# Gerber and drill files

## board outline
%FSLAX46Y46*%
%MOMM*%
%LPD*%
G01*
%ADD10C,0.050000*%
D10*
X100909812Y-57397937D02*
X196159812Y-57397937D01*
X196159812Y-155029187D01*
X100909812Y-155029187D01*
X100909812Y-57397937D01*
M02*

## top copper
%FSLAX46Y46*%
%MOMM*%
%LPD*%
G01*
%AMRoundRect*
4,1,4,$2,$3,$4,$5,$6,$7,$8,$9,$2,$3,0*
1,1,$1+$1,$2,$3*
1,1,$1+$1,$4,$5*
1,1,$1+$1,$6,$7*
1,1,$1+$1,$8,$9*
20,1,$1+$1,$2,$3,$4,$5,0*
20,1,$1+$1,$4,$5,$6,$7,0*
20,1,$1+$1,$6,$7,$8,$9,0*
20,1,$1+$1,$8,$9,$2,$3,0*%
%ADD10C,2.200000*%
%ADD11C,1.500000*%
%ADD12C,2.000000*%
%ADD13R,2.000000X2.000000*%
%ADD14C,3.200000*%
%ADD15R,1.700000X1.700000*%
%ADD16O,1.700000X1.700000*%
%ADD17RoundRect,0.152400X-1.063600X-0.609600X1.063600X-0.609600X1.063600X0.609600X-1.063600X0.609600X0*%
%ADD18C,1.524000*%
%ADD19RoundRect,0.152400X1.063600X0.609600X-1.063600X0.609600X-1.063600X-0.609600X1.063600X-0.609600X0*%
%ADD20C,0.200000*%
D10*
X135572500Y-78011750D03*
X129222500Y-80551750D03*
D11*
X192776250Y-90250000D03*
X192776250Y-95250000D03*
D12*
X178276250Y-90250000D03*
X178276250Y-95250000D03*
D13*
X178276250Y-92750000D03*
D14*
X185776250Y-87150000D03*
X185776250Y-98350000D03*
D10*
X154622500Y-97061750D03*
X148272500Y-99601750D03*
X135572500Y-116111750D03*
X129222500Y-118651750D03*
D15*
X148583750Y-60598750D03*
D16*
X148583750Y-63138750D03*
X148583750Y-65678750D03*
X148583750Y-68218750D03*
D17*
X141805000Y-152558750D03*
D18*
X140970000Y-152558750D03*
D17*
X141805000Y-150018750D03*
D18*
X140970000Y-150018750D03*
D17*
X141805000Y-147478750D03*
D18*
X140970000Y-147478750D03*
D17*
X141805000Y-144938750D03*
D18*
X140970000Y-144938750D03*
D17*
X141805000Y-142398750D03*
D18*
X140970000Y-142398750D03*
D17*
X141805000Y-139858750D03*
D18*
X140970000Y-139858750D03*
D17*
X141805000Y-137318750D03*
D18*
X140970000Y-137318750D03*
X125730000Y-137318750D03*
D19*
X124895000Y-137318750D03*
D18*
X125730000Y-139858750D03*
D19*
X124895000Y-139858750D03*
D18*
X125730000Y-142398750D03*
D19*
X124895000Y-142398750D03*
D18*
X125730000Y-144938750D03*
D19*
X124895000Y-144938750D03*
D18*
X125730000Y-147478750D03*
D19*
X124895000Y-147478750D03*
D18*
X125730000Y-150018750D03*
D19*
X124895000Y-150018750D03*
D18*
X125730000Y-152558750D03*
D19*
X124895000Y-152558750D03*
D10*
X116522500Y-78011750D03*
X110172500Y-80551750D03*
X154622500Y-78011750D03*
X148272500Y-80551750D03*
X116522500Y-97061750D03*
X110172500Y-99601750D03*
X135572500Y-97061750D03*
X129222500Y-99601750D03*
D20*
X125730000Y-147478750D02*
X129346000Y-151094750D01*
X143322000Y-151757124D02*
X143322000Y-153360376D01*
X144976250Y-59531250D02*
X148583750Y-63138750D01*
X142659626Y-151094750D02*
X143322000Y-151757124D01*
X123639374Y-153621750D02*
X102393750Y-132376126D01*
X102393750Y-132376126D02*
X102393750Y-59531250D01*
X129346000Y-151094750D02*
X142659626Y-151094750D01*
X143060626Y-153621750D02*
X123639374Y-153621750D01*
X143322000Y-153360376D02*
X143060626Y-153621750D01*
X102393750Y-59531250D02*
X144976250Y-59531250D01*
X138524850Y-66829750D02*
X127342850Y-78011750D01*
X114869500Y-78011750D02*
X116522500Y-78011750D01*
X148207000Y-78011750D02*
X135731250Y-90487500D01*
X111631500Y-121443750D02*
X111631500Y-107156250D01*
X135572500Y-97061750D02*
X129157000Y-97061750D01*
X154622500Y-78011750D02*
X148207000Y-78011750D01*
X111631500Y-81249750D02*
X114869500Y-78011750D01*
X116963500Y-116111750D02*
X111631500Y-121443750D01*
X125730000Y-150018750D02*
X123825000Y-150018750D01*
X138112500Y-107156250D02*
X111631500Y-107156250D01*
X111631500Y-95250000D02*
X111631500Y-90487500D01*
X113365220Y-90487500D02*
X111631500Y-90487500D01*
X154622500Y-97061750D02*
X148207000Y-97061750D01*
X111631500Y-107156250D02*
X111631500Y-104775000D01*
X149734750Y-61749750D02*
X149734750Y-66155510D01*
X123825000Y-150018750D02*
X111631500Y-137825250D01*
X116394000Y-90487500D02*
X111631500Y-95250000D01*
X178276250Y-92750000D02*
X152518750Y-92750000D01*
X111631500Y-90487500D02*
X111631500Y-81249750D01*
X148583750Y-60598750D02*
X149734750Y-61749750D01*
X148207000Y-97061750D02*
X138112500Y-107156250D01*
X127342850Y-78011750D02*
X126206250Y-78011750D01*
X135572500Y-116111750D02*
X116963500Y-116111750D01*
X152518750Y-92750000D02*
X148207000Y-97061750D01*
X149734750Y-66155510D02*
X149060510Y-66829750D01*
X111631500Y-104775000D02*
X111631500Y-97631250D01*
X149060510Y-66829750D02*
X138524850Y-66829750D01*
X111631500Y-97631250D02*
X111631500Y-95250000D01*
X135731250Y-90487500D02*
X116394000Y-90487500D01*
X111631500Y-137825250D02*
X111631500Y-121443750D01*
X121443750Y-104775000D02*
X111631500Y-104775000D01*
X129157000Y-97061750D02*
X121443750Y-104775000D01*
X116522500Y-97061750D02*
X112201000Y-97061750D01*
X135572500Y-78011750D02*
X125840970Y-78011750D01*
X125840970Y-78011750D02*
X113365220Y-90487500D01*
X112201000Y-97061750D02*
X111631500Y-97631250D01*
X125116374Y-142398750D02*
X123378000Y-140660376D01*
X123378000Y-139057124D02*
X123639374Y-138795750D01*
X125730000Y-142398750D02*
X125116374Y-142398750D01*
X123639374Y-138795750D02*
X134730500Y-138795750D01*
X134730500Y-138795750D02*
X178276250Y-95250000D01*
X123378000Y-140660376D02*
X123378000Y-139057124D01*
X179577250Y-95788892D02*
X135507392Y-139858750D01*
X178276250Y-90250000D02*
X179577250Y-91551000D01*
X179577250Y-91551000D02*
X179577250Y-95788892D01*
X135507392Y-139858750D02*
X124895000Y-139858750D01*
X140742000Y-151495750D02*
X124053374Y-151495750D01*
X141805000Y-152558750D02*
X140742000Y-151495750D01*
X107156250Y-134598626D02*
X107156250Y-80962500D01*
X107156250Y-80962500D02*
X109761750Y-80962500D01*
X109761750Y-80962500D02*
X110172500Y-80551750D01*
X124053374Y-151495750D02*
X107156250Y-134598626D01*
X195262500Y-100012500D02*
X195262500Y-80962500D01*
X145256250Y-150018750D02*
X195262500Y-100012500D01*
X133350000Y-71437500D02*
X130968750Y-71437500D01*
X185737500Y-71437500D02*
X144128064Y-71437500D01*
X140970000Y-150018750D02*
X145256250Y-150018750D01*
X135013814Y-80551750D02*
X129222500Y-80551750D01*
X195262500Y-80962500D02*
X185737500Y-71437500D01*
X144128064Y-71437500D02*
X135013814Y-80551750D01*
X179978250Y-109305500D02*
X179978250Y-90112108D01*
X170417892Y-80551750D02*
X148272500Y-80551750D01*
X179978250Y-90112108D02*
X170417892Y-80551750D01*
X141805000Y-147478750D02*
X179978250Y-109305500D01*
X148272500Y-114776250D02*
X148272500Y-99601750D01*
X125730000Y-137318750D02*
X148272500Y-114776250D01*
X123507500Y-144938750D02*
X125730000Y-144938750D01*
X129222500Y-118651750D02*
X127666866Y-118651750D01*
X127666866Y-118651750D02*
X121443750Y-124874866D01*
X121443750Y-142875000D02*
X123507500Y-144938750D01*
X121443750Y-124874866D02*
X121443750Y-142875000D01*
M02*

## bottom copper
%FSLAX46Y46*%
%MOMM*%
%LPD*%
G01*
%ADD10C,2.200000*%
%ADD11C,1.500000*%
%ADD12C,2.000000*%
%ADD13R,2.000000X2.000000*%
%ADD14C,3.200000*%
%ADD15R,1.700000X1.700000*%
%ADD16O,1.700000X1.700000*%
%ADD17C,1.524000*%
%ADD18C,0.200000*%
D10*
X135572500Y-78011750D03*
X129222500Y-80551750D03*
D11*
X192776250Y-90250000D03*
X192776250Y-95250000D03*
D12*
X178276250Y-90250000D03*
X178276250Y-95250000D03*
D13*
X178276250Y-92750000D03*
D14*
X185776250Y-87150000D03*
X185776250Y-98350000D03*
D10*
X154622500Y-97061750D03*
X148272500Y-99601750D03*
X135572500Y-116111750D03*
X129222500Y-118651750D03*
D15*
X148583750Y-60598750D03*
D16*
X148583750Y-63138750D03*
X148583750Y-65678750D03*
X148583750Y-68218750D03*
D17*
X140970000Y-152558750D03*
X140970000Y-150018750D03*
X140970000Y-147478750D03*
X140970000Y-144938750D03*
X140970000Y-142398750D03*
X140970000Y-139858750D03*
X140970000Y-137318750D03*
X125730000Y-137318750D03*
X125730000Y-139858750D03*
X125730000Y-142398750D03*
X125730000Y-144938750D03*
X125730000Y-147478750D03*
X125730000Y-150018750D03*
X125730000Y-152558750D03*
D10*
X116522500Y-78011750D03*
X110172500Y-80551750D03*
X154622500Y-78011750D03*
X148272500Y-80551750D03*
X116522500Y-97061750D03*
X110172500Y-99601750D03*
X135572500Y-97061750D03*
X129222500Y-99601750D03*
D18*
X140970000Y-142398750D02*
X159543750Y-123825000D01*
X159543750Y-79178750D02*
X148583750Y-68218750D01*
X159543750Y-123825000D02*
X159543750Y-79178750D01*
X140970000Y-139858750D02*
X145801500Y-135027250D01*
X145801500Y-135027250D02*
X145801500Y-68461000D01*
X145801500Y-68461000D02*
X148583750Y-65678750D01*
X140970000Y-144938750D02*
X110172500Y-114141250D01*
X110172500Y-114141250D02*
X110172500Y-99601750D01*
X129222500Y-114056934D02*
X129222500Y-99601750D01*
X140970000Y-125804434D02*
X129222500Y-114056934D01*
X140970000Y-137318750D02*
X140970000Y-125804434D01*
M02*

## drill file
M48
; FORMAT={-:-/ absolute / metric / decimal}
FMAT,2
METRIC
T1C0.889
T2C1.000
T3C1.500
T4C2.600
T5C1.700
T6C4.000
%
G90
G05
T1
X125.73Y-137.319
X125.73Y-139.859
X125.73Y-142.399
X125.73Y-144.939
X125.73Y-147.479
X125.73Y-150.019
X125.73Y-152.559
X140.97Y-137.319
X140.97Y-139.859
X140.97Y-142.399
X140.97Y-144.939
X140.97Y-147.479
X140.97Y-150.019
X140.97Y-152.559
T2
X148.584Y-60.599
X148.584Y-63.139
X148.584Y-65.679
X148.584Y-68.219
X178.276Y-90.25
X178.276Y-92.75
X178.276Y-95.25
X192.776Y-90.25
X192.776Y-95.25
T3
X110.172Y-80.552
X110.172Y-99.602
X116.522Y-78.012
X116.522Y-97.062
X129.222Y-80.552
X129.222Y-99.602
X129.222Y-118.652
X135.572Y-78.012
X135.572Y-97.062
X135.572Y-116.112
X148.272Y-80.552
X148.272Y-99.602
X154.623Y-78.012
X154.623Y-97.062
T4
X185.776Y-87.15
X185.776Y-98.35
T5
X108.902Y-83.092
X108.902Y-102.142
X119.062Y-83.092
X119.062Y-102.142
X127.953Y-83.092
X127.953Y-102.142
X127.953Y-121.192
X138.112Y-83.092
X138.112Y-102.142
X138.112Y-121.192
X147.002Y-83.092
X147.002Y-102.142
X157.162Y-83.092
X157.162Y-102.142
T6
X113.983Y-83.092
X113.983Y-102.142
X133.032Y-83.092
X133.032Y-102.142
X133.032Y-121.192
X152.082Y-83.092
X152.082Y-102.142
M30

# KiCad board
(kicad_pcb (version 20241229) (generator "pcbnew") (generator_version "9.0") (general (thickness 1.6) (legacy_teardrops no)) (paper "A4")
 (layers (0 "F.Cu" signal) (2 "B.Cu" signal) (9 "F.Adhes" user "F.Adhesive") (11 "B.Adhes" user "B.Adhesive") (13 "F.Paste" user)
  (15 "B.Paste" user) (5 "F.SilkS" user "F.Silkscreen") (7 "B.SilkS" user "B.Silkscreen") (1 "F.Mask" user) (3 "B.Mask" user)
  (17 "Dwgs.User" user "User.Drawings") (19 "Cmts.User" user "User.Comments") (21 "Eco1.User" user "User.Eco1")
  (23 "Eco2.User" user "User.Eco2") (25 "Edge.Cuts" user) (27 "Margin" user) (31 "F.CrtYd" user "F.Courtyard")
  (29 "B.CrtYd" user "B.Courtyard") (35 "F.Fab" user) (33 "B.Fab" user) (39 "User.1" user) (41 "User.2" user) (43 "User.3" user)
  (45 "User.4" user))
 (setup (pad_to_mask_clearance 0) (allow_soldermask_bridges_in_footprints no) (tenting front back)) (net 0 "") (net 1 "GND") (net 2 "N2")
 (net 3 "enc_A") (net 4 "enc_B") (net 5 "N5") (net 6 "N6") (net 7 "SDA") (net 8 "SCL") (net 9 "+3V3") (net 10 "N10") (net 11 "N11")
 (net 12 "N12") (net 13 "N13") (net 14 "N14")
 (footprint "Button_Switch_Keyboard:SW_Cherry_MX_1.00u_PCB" (layer "F.Cu") (at 135.5725 78.01175)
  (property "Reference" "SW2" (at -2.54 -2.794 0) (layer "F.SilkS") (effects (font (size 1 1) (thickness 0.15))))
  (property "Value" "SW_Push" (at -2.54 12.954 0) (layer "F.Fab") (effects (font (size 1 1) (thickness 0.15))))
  (pad "" np_thru_hole circle (at -7.62 5.08) (size 1.7 1.7) (drill 1.7) (layers "*.Cu" "*.Mask"))
  (pad "" np_thru_hole circle (at -2.54 5.08) (size 4 4) (drill 4) (layers "*.Cu" "*.Mask"))
  (pad "" np_thru_hole circle (at 2.54 5.08) (size 1.7 1.7) (drill 1.7) (layers "*.Cu" "*.Mask"))
  (pad "1" thru_hole circle (at 0 0) (size 2.2 2.2) (drill 1.5) (layers "*.Cu" "*.Mask") (remove_unused_layers no) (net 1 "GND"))
  (pad "2" thru_hole circle (at -6.35 2.54) (size 2.2 2.2) (drill 1.5) (layers "*.Cu" "*.Mask") (remove_unused_layers no) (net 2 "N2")))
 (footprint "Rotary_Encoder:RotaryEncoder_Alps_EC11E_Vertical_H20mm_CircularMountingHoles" (layer "F.Cu") (at 178.27625 90.25)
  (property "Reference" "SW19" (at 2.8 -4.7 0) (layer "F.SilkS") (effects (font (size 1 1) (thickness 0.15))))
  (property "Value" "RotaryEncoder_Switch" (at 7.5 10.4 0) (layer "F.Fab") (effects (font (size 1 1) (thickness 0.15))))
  (pad "" thru_hole circle (at 14.5 0) (size 1.5 1.5) (drill 1) (layers "*.Cu" "*.Mask") (remove_unused_layers no))
  (pad "" thru_hole circle (at 14.5 5) (size 1.5 1.5) (drill 1) (layers "*.Cu" "*.Mask") (remove_unused_layers no))
  (pad "A" thru_hole circle (at 0 0) (size 2 2) (drill 1) (layers "*.Cu" "*.Mask") (remove_unused_layers no) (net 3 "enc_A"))
  (pad "B" thru_hole circle (at 0 5) (size 2 2) (drill 1) (layers "*.Cu" "*.Mask") (remove_unused_layers no) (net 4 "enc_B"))
  (pad "C" thru_hole rect (at 0 2.5) (size 2 2) (drill 1) (layers "*.Cu" "*.Mask") (remove_unused_layers no) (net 1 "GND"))
  (pad "MP" thru_hole circle (at 7.5 -3.1) (size 3.2 3.2) (drill 2.6) (layers "*.Cu" "*.Mask") (remove_unused_layers no))
  (pad "MP" thru_hole circle (at 7.5 8.1) (size 3.2 3.2) (drill 2.6) (layers "*.Cu" "*.Mask") (remove_unused_layers no)))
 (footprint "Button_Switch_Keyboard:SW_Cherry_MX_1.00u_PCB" (layer "F.Cu") (at 154.6225 97.06175)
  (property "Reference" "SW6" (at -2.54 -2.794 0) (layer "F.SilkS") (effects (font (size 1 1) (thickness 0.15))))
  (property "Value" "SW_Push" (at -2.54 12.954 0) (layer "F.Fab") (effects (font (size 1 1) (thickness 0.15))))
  (pad "" np_thru_hole circle (at -7.62 5.08) (size 1.7 1.7) (drill 1.7) (layers "*.Cu" "*.Mask"))
  (pad "" np_thru_hole circle (at -2.54 5.08) (size 4 4) (drill 4) (layers "*.Cu" "*.Mask"))
  (pad "" np_thru_hole circle (at 2.54 5.08) (size 1.7 1.7) (drill 1.7) (layers "*.Cu" "*.Mask"))
  (pad "1" thru_hole circle (at 0 0) (size 2.2 2.2) (drill 1.5) (layers "*.Cu" "*.Mask") (remove_unused_layers no) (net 1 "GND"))
  (pad "2" thru_hole circle (at -6.35 2.54) (size 2.2 2.2) (drill 1.5) (layers "*.Cu" "*.Mask") (remove_unused_layers no) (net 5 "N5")))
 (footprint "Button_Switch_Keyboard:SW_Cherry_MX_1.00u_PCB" (layer "F.Cu") (at 135.5725 116.11175)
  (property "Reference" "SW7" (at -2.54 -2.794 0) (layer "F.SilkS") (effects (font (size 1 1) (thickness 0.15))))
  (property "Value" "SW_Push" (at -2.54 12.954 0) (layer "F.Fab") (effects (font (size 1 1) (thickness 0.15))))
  (pad "" np_thru_hole circle (at -7.62 5.08) (size 1.7 1.7) (drill 1.7) (layers "*.Cu" "*.Mask"))
  (pad "" np_thru_hole circle (at -2.54 5.08) (size 4 4) (drill 4) (layers "*.Cu" "*.Mask"))
  (pad "" np_thru_hole circle (at 2.54 5.08) (size 1.7 1.7) (drill 1.7) (layers "*.Cu" "*.Mask"))
  (pad "1" thru_hole circle (at 0 0) (size 2.2 2.2) (drill 1.5) (layers "*.Cu" "*.Mask") (remove_unused_layers no) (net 1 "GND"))
  (pad "2" thru_hole circle (at -6.35 2.54) (size 2.2 2.2) (drill 1.5) (layers "*.Cu" "*.Mask") (remove_unused_layers no) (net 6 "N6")))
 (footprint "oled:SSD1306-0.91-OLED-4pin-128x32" (layer "F.Cu") (at 112.08375 58.40875)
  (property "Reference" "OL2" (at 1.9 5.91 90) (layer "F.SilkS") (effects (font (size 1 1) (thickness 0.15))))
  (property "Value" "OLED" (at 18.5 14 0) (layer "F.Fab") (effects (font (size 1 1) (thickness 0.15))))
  (pad "1" thru_hole rect (at 36.5 2.19) (size 1.7 1.7) (drill 1) (layers "*.Cu" "*.Mask") (remove_unused_layers no) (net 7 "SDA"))
  (pad "2" thru_hole oval (at 36.5 4.73) (size 1.7 1.7) (drill 1) (layers "*.Cu" "*.Mask") (remove_unused_layers no) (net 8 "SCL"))
  (pad "3" thru_hole oval (at 36.5 7.27) (size 1.7 1.7) (drill 1) (layers "*.Cu" "*.Mask") (remove_unused_layers no) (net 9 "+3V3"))
  (pad "4" thru_hole oval (at 36.5 9.81) (size 1.7 1.7) (drill 1) (layers "*.Cu" "*.Mask") (remove_unused_layers no) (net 1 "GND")))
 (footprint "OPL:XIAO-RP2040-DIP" (layer "F.Cu") (at 133.35 144.93875 180)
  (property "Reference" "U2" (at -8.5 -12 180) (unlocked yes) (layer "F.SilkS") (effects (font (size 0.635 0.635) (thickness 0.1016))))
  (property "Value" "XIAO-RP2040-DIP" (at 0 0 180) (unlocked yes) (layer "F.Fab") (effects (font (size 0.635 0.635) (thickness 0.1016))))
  (pad "1" smd roundrect (at -8.455 -7.62) (size 2.432 1.524) (layers "F.Cu" "F.Mask") (roundrect_rratio 0.1) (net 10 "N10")
   (thermal_bridge_angle 45))
  (pad "1" thru_hole circle (at -7.62 -7.62) (size 1.524 1.524) (drill 0.889) (layers "*.Cu" "*.Mask") (remove_unused_layers no)
   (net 10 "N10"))
  (pad "2" smd roundrect (at -8.455 -5.08) (size 2.432 1.524) (layers "F.Cu" "F.Mask") (roundrect_rratio 0.1) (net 2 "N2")
   (thermal_bridge_angle 45))
  (pad "2" thru_hole circle (at -7.62 -5.08) (size 1.524 1.524) (drill 0.889) (layers "*.Cu" "*.Mask") (remove_unused_layers no)
   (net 2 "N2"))
  (pad "3" smd roundrect (at -8.455 -2.54) (size 2.432 1.524) (layers "F.Cu" "F.Mask") (roundrect_rratio 0.1) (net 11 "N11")
   (thermal_bridge_angle 45))
  (pad "3" thru_hole circle (at -7.62 -2.54) (size 1.524 1.524) (drill 0.889) (layers "*.Cu" "*.Mask") (remove_unused_layers no)
   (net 11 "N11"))
  (pad "4" smd roundrect (at -8.455 0) (size 2.432 1.524) (layers "F.Cu" "F.Mask") (roundrect_rratio 0.1) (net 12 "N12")
   (thermal_bridge_angle 45))
  (pad "4" thru_hole circle (at -7.62 0) (size 1.524 1.524) (drill 0.889) (layers "*.Cu" "*.Mask") (remove_unused_layers no) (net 12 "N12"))
  (pad "5" smd roundrect (at -8.455 2.54) (size 2.432 1.524) (layers "F.Cu" "F.Mask") (roundrect_rratio 0.1) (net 7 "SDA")
   (thermal_bridge_angle 45))
  (pad "5" thru_hole circle (at -7.62 2.54) (size 1.524 1.524) (drill 0.889) (layers "*.Cu" "*.Mask") (remove_unused_layers no)
   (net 7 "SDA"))
  (pad "6" smd roundrect (at -8.455 5.08) (size 2.432 1.524) (layers "F.Cu" "F.Mask") (roundrect_rratio 0.1) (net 8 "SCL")
   (thermal_bridge_angle 45))
  (pad "6" thru_hole circle (at -7.62 5.08) (size 1.524 1.524) (drill 0.889) (layers "*.Cu" "*.Mask") (remove_unused_layers no)
   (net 8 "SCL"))
  (pad "7" smd roundrect (at -8.455 7.62) (size 2.432 1.524) (layers "F.Cu" "F.Mask") (roundrect_rratio 0.1) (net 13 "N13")
   (thermal_bridge_angle 45))
  (pad "7" thru_hole circle (at -7.62 7.62) (size 1.524 1.524) (drill 0.889) (layers "*.Cu" "*.Mask") (remove_unused_layers no)
   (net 13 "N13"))
  (pad "8" thru_hole circle (at 7.62 7.62 180) (size 1.524 1.524) (drill 0.889) (layers "*.Cu" "*.Mask") (remove_unused_layers no)
   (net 5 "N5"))
  (pad "8" smd roundrect (at 8.455 7.62 180) (size 2.432 1.524) (layers "F.Cu" "F.Mask") (roundrect_rratio 0.1) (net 5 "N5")
   (thermal_bridge_angle 45))
  (pad "9" thru_hole circle (at 7.62 5.08 180) (size 1.524 1.524) (drill 0.889) (layers "*.Cu" "*.Mask") (remove_unused_layers no)
   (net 3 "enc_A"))
  (pad "9" smd roundrect (at 8.455 5.08 180) (size 2.432 1.524) (layers "F.Cu" "F.Mask") (roundrect_rratio 0.1) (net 3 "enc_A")
   (thermal_bridge_angle 45))
  (pad "10" thru_hole circle (at 7.62 2.54 180) (size 1.524 1.524) (drill 0.889) (layers "*.Cu" "*.Mask") (remove_unused_layers no)
   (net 4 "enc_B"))
  (pad "10" smd roundrect (at 8.455 2.54 180) (size 2.432 1.524) (layers "F.Cu" "F.Mask") (roundrect_rratio 0.1) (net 4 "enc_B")
   (thermal_bridge_angle 45))
  (pad "11" thru_hole circle (at 7.62 0 180) (size 1.524 1.524) (drill 0.889) (layers "*.Cu" "*.Mask") (remove_unused_layers no)
   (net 6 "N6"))
  (pad "11" smd roundrect (at 8.455 0 180) (size 2.432 1.524) (layers "F.Cu" "F.Mask") (roundrect_rratio 0.1) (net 6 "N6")
   (thermal_bridge_angle 45))
  (pad "12" thru_hole circle (at 7.62 -2.54 180) (size 1.524 1.524) (drill 0.889) (layers "*.Cu" "*.Mask") (remove_unused_layers no)
   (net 9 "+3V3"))
  (pad "12" smd roundrect (at 8.455 -2.54 180) (size 2.432 1.524) (layers "F.Cu" "F.Mask") (roundrect_rratio 0.1) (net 9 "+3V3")
   (thermal_bridge_angle 45))
  (pad "13" thru_hole circle (at 7.62 -5.08 180) (size 1.524 1.524) (drill 0.889) (layers "*.Cu" "*.Mask") (remove_unused_layers no)
   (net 1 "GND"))
  (pad "13" smd roundrect (at 8.455 -5.08 180) (size 2.432 1.524) (layers "F.Cu" "F.Mask") (roundrect_rratio 0.1) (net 1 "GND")
   (thermal_bridge_angle 45))
  (pad "14" thru_hole circle (at 7.62 -7.62 180) (size 1.524 1.524) (drill 0.889) (layers "*.Cu" "*.Mask") (remove_unused_layers no)
   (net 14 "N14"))
  (pad "14" smd roundrect (at 8.455 -7.62 180) (size 2.432 1.524) (layers "F.Cu" "F.Mask") (roundrect_rratio 0.1) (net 14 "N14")
   (thermal_bridge_angle 45)))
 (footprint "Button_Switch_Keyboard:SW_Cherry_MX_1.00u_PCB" (layer "F.Cu") (at 116.5225 78.01175)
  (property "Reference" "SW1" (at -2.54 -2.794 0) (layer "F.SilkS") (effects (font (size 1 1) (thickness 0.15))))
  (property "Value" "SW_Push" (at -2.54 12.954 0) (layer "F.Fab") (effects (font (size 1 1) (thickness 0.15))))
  (pad "" np_thru_hole circle (at -7.62 5.08) (size 1.7 1.7) (drill 1.7) (layers "*.Cu" "*.Mask"))
  (pad "" np_thru_hole circle (at -2.54 5.08) (size 4 4) (drill 4) (layers "*.Cu" "*.Mask"))
  (pad "" np_thru_hole circle (at 2.54 5.08) (size 1.7 1.7) (drill 1.7) (layers "*.Cu" "*.Mask"))
  (pad "1" thru_hole circle (at 0 0) (size 2.2 2.2) (drill 1.5) (layers "*.Cu" "*.Mask") (remove_unused_layers no) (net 1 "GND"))
  (pad "2" thru_hole circle (at -6.35 2.54) (size 2.2 2.2) (drill 1.5) (layers "*.Cu" "*.Mask") (remove_unused_layers no) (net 10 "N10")))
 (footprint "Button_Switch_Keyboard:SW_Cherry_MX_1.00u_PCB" (layer "F.Cu") (at 154.6225 78.01175)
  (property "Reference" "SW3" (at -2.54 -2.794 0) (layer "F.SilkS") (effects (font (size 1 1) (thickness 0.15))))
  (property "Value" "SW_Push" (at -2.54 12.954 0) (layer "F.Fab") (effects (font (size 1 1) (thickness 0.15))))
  (pad "" np_thru_hole circle (at -7.62 5.08) (size 1.7 1.7) (drill 1.7) (layers "*.Cu" "*.Mask"))
  (pad "" np_thru_hole circle (at -2.54 5.08) (size 4 4) (drill 4) (layers "*.Cu" "*.Mask"))
  (pad "" np_thru_hole circle (at 2.54 5.08) (size 1.7 1.7) (drill 1.7) (layers "*.Cu" "*.Mask"))
  (pad "1" thru_hole circle (at 0 0) (size 2.2 2.2) (drill 1.5) (layers "*.Cu" "*.Mask") (remove_unused_layers no) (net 1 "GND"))
  (pad "2" thru_hole circle (at -6.35 2.54) (size 2.2 2.2) (drill 1.5) (layers "*.Cu" "*.Mask") (remove_unused_layers no) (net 11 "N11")))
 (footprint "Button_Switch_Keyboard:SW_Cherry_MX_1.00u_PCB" (layer "F.Cu") (at 116.5225 97.06175)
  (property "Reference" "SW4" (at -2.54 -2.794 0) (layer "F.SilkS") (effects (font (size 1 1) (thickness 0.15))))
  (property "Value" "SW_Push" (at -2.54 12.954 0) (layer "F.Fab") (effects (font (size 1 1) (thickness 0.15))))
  (pad "" np_thru_hole circle (at -7.62 5.08) (size 1.7 1.7) (drill 1.7) (layers "*.Cu" "*.Mask"))
  (pad "" np_thru_hole circle (at -2.54 5.08) (size 4 4) (drill 4) (layers "*.Cu" "*.Mask"))
  (pad "" np_thru_hole circle (at 2.54 5.08) (size 1.7 1.7) (drill 1.7) (layers "*.Cu" "*.Mask"))
  (pad "1" thru_hole circle (at 0 0) (size 2.2 2.2) (drill 1.5) (layers "*.Cu" "*.Mask") (remove_unused_layers no) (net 1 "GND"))
  (pad "2" thru_hole circle (at -6.35 2.54) (size 2.2 2.2) (drill 1.5) (layers "*.Cu" "*.Mask") (remove_unused_layers no) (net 12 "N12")))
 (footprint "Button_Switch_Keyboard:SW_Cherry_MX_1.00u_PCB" (layer "F.Cu") (at 135.5725 97.06175)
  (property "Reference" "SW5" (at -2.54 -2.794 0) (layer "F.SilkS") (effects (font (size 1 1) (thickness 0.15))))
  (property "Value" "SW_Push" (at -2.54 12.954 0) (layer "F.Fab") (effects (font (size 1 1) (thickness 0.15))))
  (pad "" np_thru_hole circle (at -7.62 5.08) (size 1.7 1.7) (drill 1.7) (layers "*.Cu" "*.Mask"))
  (pad "" np_thru_hole circle (at -2.54 5.08) (size 4 4) (drill 4) (layers "*.Cu" "*.Mask"))
  (pad "" np_thru_hole circle (at 2.54 5.08) (size 1.7 1.7) (drill 1.7) (layers "*.Cu" "*.Mask"))
  (pad "1" thru_hole circle (at 0 0) (size 2.2 2.2) (drill 1.5) (layers "*.Cu" "*.Mask") (remove_unused_layers no) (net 1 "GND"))
  (pad "2" thru_hole circle (at -6.35 2.54) (size 2.2 2.2) (drill 1.5) (layers "*.Cu" "*.Mask") (remove_unused_layers no) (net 13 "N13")))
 (gr_rect (start 100.909812 57.397937) (end 196.159812 155.029187) (stroke (width 0.05) (type default)) (fill no) (layer "Edge.Cuts"))
 (segment (start 140.97 142.39875) (end 159.54375 123.825) (width 0.2) (layer "B.Cu") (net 7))
 (segment (start 159.54375 79.17875) (end 148.58375 68.21875) (width 0.2) (layer "B.Cu") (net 7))
 (segment (start 159.54375 123.825) (end 159.54375 79.17875) (width 0.2) (layer "B.Cu") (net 7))
 (segment (start 125.73 147.47875) (end 129.346 151.09475) (width 0.2) (layer "F.Cu") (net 9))
 (segment (start 143.322 151.757124) (end 143.322 153.360376) (width 0.2) (layer "F.Cu") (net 9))
 (segment (start 144.97625 59.53125) (end 148.58375 63.13875) (width 0.2) (layer "F.Cu") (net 9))
 (segment (start 142.659626 151.09475) (end 143.322 151.757124) (width 0.2) (layer "F.Cu") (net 9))
 (segment (start 123.639374 153.62175) (end 102.39375 132.376126) (width 0.2) (layer "F.Cu") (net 9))
 (segment (start 102.39375 132.376126) (end 102.39375 59.53125) (width 0.2) (layer "F.Cu") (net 9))
 (segment (start 129.346 151.09475) (end 142.659626 151.09475) (width 0.2) (layer "F.Cu") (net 9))
 (segment (start 143.060626 153.62175) (end 123.639374 153.62175) (width 0.2) (layer "F.Cu") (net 9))
 (segment (start 143.322 153.360376) (end 143.060626 153.62175) (width 0.2) (layer "F.Cu") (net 9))
 (segment (start 102.39375 59.53125) (end 144.97625 59.53125) (width 0.2) (layer "F.Cu") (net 9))
 (segment (start 138.52485 66.82975) (end 127.34285 78.01175) (width 0.2) (layer "F.Cu") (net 1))
 (segment (start 114.8695 78.01175) (end 116.5225 78.01175) (width 0.2) (layer "F.Cu") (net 1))
 (segment (start 148.207 78.01175) (end 135.73125 90.4875) (width 0.2) (layer "F.Cu") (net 1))
 (segment (start 111.6315 121.44375) (end 111.6315 107.15625) (width 0.2) (layer "F.Cu") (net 1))
 (segment (start 135.5725 97.06175) (end 129.157 97.06175) (width 0.2) (layer "F.Cu") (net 1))
 (segment (start 154.6225 78.01175) (end 148.207 78.01175) (width 0.2) (layer "F.Cu") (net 1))
 (segment (start 111.6315 81.24975) (end 114.8695 78.01175) (width 0.2) (layer "F.Cu") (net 1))
 (segment (start 116.9635 116.11175) (end 111.6315 121.44375) (width 0.2) (layer "F.Cu") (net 1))
 (segment (start 125.73 150.01875) (end 123.825 150.01875) (width 0.2) (layer "F.Cu") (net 1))
 (segment (start 138.1125 107.15625) (end 111.6315 107.15625) (width 0.2) (layer "F.Cu") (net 1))
 (segment (start 111.6315 95.25) (end 111.6315 90.4875) (width 0.2) (layer "F.Cu") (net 1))
 (segment (start 113.36522 90.4875) (end 111.6315 90.4875) (width 0.2) (layer "F.Cu") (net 1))
 (segment (start 154.6225 97.06175) (end 148.207 97.06175) (width 0.2) (layer "F.Cu") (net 1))
 (segment (start 111.6315 107.15625) (end 111.6315 104.775) (width 0.2) (layer "F.Cu") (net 1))
 (segment (start 149.73475 61.74975) (end 149.73475 66.15551) (width 0.2) (layer "F.Cu") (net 1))
 (segment (start 123.825 150.01875) (end 111.6315 137.82525) (width 0.2) (layer "F.Cu") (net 1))
 (segment (start 116.394 90.4875) (end 111.6315 95.25) (width 0.2) (layer "F.Cu") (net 1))
 (segment (start 178.27625 92.75) (end 152.51875 92.75) (width 0.2) (layer "F.Cu") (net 1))
 (segment (start 111.6315 90.4875) (end 111.6315 81.24975) (width 0.2) (layer "F.Cu") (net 1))
 (segment (start 148.58375 60.59875) (end 149.73475 61.74975) (width 0.2) (layer "F.Cu") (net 1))
 (segment (start 148.207 97.06175) (end 138.1125 107.15625) (width 0.2) (layer "F.Cu") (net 1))
 (segment (start 127.34285 78.01175) (end 126.20625 78.01175) (width 0.2) (layer "F.Cu") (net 1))
 (segment (start 135.5725 116.11175) (end 116.9635 116.11175) (width 0.2) (layer "F.Cu") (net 1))
 (segment (start 152.51875 92.75) (end 148.207 97.06175) (width 0.2) (layer "F.Cu") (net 1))
 (segment (start 149.73475 66.15551) (end 149.06051 66.82975) (width 0.2) (layer "F.Cu") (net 1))
 (segment (start 111.6315 104.775) (end 111.6315 97.63125) (width 0.2) (layer "F.Cu") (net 1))
 (segment (start 149.06051 66.82975) (end 138.52485 66.82975) (width 0.2) (layer "F.Cu") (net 1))
 (segment (start 111.6315 97.63125) (end 111.6315 95.25) (width 0.2) (layer "F.Cu") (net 1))
 (segment (start 135.73125 90.4875) (end 116.394 90.4875) (width 0.2) (layer "F.Cu") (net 1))
 (segment (start 111.6315 137.82525) (end 111.6315 121.44375) (width 0.2) (layer "F.Cu") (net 1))
 (segment (start 121.44375 104.775) (end 111.6315 104.775) (width 0.2) (layer "F.Cu") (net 1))
 (segment (start 129.157 97.06175) (end 121.44375 104.775) (width 0.2) (layer "F.Cu") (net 1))
 (segment (start 116.5225 97.06175) (end 112.201 97.06175) (width 0.2) (layer "F.Cu") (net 1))
 (segment (start 135.5725 78.01175) (end 125.84097 78.01175) (width 0.2) (layer "F.Cu") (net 1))
 (segment (start 125.84097 78.01175) (end 113.36522 90.4875) (width 0.2) (layer "F.Cu") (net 1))
 (segment (start 112.201 97.06175) (end 111.6315 97.63125) (width 0.2) (layer "F.Cu") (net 1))
 (segment (start 140.97 139.85875) (end 145.8015 135.02725) (width 0.2) (layer "B.Cu") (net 8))
 (segment (start 145.8015 135.02725) (end 145.8015 68.461) (width 0.2) (layer "B.Cu") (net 8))
 (segment (start 145.8015 68.461) (end 148.58375 65.67875) (width 0.2) (layer "B.Cu") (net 8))
 (segment (start 125.116374 142.39875) (end 123.378 140.660376) (width 0.2) (layer "F.Cu") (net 4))
 (segment (start 123.378 139.057124) (end 123.639374 138.79575) (width 0.2) (layer "F.Cu") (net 4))
 (segment (start 125.73 142.39875) (end 125.116374 142.39875) (width 0.2) (layer "F.Cu") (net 4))
 (segment (start 123.639374 138.79575) (end 134.7305 138.79575) (width 0.2) (layer "F.Cu") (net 4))
 (segment (start 134.7305 138.79575) (end 178.27625 95.25) (width 0.2) (layer "F.Cu") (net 4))
 (segment (start 123.378 140.660376) (end 123.378 139.057124) (width 0.2) (layer "F.Cu") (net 4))
 (segment (start 179.57725 95.788892) (end 135.507392 139.85875) (width 0.2) (layer "F.Cu") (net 3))
 (segment (start 178.27625 90.25) (end 179.57725 91.551) (width 0.2) (layer "F.Cu") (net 3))
 (segment (start 179.57725 91.551) (end 179.57725 95.788892) (width 0.2) (layer "F.Cu") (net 3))
 (segment (start 135.507392 139.85875) (end 124.895 139.85875) (width 0.2) (layer "F.Cu") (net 3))
 (segment (start 140.742 151.49575) (end 124.053374 151.49575) (width 0.2) (layer "F.Cu") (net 10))
 (segment (start 141.805 152.55875) (end 140.742 151.49575) (width 0.2) (layer "F.Cu") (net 10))
 (segment (start 107.15625 134.598626) (end 107.15625 80.9625) (width 0.2) (layer "F.Cu") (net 10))
 (segment (start 107.15625 80.9625) (end 109.76175 80.9625) (width 0.2) (layer "F.Cu") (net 10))
 (segment (start 109.76175 80.9625) (end 110.1725 80.55175) (width 0.2) (layer "F.Cu") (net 10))
 (segment (start 124.053374 151.49575) (end 107.15625 134.598626) (width 0.2) (layer "F.Cu") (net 10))
 (segment (start 195.2625 100.0125) (end 195.2625 80.9625) (width 0.2) (layer "F.Cu") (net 2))
 (segment (start 145.25625 150.01875) (end 195.2625 100.0125) (width 0.2) (layer "F.Cu") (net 2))
 (segment (start 133.35 71.4375) (end 130.96875 71.4375) (width 0.2) (layer "F.Cu") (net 2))
 (segment (start 185.7375 71.4375) (end 144.128064 71.4375) (width 0.2) (layer "F.Cu") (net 2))
 (segment (start 140.97 150.01875) (end 145.25625 150.01875) (width 0.2) (layer "F.Cu") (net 2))
 (segment (start 135.013814 80.55175) (end 129.2225 80.55175) (width 0.2) (layer "F.Cu") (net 2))
 (segment (start 195.2625 80.9625) (end 185.7375 71.4375) (width 0.2) (layer "F.Cu") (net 2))
 (segment (start 144.128064 71.4375) (end 135.013814 80.55175) (width 0.2) (layer "F.Cu") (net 2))
 (segment (start 179.97825 109.3055) (end 179.97825 90.112108) (width 0.2) (layer "F.Cu") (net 11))
 (segment (start 170.417892 80.55175) (end 148.2725 80.55175) (width 0.2) (layer "F.Cu") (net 11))
 (segment (start 179.97825 90.112108) (end 170.417892 80.55175) (width 0.2) (layer "F.Cu") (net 11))
 (segment (start 141.805 147.47875) (end 179.97825 109.3055) (width 0.2) (layer "F.Cu") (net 11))
 (segment (start 140.97 144.93875) (end 110.1725 114.14125) (width 0.2) (layer "B.Cu") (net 12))
 (segment (start 110.1725 114.14125) (end 110.1725 99.60175) (width 0.2) (layer "B.Cu") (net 12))
 (segment (start 129.2225 114.056934) (end 129.2225 99.60175) (width 0.2) (layer "B.Cu") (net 13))
 (segment (start 140.97 125.804434) (end 129.2225 114.056934) (width 0.2) (layer "B.Cu") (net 13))
 (segment (start 140.97 137.31875) (end 140.97 125.804434) (width 0.2) (layer "B.Cu") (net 13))
 (segment (start 148.2725 114.77625) (end 148.2725 99.60175) (width 0.2) (layer "F.Cu") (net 5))
 (segment (start 125.73 137.31875) (end 148.2725 114.77625) (width 0.2) (layer "F.Cu") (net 5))
 (segment (start 123.5075 144.93875) (end 125.73 144.93875) (width 0.2) (layer "F.Cu") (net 6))
 (segment (start 129.2225 118.65175) (end 127.666866 118.65175) (width 0.2) (layer "F.Cu") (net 6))
 (segment (start 127.666866 118.65175) (end 121.44375 124.874866) (width 0.2) (layer "F.Cu") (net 6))
 (segment (start 121.44375 142.875) (end 123.5075 144.93875) (width 0.2) (layer "F.Cu") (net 6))
 (segment (start 121.44375 124.874866) (end 121.44375 142.875) (width 0.2) (layer "F.Cu") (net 6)))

